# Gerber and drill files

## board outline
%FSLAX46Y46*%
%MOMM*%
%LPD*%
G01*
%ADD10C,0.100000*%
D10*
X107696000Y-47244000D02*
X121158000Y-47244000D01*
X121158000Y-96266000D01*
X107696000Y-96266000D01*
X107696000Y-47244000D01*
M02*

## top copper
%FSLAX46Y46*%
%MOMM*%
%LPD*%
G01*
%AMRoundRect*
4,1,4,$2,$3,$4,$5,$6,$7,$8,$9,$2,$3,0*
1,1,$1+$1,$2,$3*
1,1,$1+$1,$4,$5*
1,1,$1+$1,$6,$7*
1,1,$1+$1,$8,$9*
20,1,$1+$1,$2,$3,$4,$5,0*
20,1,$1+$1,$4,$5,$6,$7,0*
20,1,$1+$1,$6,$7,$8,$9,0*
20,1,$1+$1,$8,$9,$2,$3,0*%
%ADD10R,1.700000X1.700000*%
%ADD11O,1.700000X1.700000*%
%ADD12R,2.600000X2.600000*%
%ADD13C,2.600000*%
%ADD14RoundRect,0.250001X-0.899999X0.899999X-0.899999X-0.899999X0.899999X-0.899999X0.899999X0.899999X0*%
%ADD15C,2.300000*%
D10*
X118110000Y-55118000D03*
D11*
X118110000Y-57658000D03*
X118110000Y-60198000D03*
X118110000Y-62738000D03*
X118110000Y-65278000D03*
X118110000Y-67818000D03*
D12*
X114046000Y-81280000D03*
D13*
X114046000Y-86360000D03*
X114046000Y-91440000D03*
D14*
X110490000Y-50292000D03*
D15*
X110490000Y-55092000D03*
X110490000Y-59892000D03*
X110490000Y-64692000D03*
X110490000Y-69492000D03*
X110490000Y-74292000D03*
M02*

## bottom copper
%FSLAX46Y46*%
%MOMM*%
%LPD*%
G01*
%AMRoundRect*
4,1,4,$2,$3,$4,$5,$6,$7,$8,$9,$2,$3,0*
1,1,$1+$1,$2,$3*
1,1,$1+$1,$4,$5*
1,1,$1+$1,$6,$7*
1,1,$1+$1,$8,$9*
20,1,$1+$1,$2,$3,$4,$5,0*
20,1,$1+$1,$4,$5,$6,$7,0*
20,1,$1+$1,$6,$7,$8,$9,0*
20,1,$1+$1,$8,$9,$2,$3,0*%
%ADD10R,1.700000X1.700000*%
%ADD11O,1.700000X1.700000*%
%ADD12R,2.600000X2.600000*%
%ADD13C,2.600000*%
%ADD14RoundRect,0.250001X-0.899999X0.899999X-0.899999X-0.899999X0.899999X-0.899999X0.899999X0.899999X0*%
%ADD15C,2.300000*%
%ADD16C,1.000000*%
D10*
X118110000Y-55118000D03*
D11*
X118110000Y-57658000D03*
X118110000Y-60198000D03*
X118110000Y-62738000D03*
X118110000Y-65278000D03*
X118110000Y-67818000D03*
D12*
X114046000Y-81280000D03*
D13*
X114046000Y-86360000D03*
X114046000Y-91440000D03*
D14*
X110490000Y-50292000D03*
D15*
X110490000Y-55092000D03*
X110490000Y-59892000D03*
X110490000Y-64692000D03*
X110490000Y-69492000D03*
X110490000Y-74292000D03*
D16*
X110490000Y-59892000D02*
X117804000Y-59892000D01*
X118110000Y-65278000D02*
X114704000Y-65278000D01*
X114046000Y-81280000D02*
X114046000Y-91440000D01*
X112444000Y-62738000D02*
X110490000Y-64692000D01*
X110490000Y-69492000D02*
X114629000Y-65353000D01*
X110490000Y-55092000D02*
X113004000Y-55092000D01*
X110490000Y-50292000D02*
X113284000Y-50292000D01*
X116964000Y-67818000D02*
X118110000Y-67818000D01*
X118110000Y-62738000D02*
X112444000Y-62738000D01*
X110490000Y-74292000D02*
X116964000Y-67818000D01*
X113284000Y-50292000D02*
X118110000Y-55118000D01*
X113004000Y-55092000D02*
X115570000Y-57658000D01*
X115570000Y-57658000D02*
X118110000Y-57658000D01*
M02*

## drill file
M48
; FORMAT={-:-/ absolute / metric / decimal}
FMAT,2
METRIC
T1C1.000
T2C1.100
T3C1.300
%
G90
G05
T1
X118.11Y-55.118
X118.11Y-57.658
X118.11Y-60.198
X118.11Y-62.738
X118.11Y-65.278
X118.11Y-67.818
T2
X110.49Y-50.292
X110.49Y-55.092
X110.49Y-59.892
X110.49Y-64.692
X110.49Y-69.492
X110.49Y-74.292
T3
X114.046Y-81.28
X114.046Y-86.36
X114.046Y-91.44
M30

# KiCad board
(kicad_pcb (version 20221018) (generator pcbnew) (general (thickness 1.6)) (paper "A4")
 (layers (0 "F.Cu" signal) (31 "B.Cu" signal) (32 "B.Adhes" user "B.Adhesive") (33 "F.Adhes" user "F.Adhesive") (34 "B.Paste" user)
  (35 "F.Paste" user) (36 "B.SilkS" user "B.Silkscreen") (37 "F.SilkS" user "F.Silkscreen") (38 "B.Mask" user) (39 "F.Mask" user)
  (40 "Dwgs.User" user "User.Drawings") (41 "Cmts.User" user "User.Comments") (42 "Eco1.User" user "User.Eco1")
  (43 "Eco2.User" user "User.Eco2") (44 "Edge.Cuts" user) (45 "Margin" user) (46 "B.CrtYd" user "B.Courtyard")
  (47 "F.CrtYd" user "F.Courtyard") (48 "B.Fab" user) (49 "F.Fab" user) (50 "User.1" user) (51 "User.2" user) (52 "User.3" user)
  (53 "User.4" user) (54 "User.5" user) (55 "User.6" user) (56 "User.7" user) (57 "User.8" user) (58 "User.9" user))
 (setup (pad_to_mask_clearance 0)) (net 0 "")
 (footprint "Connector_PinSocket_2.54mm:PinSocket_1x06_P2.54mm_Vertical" (layer "F.Cu") (at 118.11 55.118)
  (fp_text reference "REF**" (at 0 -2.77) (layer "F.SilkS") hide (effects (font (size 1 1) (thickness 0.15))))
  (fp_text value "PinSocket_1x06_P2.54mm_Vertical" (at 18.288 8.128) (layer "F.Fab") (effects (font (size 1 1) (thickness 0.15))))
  (pad "1" thru_hole rect (at 0 0) (size 1.7 1.7) (drill 1) (layers "*.Cu" "*.Mask"))
  (pad "2" thru_hole oval (at 0 2.54) (size 1.7 1.7) (drill 1) (layers "*.Cu" "*.Mask"))
  (pad "3" thru_hole oval (at 0 5.08) (size 1.7 1.7) (drill 1) (layers "*.Cu" "*.Mask"))
  (pad "4" thru_hole oval (at 0 7.62) (size 1.7 1.7) (drill 1) (layers "*.Cu" "*.Mask"))
  (pad "5" thru_hole oval (at 0 10.16) (size 1.7 1.7) (drill 1) (layers "*.Cu" "*.Mask"))
  (pad "6" thru_hole oval (at 0 12.7) (size 1.7 1.7) (drill 1) (layers "*.Cu" "*.Mask")))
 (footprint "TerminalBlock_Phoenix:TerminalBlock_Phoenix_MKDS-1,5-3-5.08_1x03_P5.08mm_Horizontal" (layer "F.Cu") (at 114.046 81.28 -90)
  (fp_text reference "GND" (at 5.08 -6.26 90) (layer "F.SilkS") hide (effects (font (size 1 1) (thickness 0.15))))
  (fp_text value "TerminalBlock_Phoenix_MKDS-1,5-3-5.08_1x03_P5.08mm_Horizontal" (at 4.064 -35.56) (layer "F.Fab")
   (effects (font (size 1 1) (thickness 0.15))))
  (pad "1" thru_hole rect (at 0 0 270) (size 2.6 2.6) (drill 1.3) (layers "*.Cu" "*.Mask"))
  (pad "2" thru_hole circle (at 5.08 0 270) (size 2.6 2.6) (drill 1.3) (layers "*.Cu" "*.Mask"))
  (pad "3" thru_hole circle (at 10.16 0 270) (size 2.6 2.6) (drill 1.3) (layers "*.Cu" "*.Mask")))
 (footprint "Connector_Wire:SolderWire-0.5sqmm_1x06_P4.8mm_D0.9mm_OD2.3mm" (layer "F.Cu") (at 110.49 50.292 -90)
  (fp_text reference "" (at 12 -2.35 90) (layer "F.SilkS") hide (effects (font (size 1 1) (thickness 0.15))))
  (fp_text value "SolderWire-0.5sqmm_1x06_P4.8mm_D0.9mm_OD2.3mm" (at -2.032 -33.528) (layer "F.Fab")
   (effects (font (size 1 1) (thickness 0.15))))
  (pad "1" thru_hole roundrect (at 0 0 270) (size 2.3 2.3) (drill 1.1) (layers "*.Cu" "*.Mask") (roundrect_rratio 0.108696087))
  (pad "2" thru_hole circle (at 4.8 0 270) (size 2.3 2.3) (drill 1.1) (layers "*.Cu" "*.Mask"))
  (pad "3" thru_hole circle (at 9.6 0 270) (size 2.3 2.3) (drill 1.1) (layers "*.Cu" "*.Mask"))
  (pad "4" thru_hole circle (at 14.4 0 270) (size 2.3 2.3) (drill 1.1) (layers "*.Cu" "*.Mask"))
  (pad "5" thru_hole circle (at 19.2 0 270) (size 2.3 2.3) (drill 1.1) (layers "*.Cu" "*.Mask"))
  (pad "6" thru_hole circle (at 24 0 270) (size 2.3 2.3) (drill 1.1) (layers "*.Cu" "*.Mask")))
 (gr_rect (start 107.696 47.244) (end 121.158 96.266) (stroke (width 0.1) (type default)) (fill none) (layer "Edge.Cuts"))
 (segment (start 110.49 59.892) (end 117.804 59.892) (width 1) (layer "B.Cu") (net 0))
 (segment (start 118.11 65.278) (end 114.704 65.278) (width 1) (layer "B.Cu") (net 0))
 (segment (start 114.046 81.28) (end 114.046 91.44) (width 1) (layer "B.Cu") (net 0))
 (segment (start 112.444 62.738) (end 110.49 64.692) (width 1) (layer "B.Cu") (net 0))
 (segment (start 110.49 69.492) (end 114.629 65.353) (width 1) (layer "B.Cu") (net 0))
 (segment (start 110.49 55.092) (end 113.004 55.092) (width 1) (layer "B.Cu") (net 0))
 (segment (start 110.49 50.292) (end 113.284 50.292) (width 1) (layer "B.Cu") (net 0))
 (segment (start 116.964 67.818) (end 118.11 67.818) (width 1) (layer "B.Cu") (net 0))
 (segment (start 118.11 62.738) (end 112.444 62.738) (width 1) (layer "B.Cu") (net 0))
 (segment (start 110.49 74.292) (end 116.964 67.818) (width 1) (layer "B.Cu") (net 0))
 (segment (start 113.284 50.292) (end 118.11 55.118) (width 1) (layer "B.Cu") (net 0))
 (segment (start 113.004 55.092) (end 115.57 57.658) (width 1) (layer "B.Cu") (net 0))
 (segment (start 115.57 57.658) (end 118.11 57.658) (width 1) (layer "B.Cu") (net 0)))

